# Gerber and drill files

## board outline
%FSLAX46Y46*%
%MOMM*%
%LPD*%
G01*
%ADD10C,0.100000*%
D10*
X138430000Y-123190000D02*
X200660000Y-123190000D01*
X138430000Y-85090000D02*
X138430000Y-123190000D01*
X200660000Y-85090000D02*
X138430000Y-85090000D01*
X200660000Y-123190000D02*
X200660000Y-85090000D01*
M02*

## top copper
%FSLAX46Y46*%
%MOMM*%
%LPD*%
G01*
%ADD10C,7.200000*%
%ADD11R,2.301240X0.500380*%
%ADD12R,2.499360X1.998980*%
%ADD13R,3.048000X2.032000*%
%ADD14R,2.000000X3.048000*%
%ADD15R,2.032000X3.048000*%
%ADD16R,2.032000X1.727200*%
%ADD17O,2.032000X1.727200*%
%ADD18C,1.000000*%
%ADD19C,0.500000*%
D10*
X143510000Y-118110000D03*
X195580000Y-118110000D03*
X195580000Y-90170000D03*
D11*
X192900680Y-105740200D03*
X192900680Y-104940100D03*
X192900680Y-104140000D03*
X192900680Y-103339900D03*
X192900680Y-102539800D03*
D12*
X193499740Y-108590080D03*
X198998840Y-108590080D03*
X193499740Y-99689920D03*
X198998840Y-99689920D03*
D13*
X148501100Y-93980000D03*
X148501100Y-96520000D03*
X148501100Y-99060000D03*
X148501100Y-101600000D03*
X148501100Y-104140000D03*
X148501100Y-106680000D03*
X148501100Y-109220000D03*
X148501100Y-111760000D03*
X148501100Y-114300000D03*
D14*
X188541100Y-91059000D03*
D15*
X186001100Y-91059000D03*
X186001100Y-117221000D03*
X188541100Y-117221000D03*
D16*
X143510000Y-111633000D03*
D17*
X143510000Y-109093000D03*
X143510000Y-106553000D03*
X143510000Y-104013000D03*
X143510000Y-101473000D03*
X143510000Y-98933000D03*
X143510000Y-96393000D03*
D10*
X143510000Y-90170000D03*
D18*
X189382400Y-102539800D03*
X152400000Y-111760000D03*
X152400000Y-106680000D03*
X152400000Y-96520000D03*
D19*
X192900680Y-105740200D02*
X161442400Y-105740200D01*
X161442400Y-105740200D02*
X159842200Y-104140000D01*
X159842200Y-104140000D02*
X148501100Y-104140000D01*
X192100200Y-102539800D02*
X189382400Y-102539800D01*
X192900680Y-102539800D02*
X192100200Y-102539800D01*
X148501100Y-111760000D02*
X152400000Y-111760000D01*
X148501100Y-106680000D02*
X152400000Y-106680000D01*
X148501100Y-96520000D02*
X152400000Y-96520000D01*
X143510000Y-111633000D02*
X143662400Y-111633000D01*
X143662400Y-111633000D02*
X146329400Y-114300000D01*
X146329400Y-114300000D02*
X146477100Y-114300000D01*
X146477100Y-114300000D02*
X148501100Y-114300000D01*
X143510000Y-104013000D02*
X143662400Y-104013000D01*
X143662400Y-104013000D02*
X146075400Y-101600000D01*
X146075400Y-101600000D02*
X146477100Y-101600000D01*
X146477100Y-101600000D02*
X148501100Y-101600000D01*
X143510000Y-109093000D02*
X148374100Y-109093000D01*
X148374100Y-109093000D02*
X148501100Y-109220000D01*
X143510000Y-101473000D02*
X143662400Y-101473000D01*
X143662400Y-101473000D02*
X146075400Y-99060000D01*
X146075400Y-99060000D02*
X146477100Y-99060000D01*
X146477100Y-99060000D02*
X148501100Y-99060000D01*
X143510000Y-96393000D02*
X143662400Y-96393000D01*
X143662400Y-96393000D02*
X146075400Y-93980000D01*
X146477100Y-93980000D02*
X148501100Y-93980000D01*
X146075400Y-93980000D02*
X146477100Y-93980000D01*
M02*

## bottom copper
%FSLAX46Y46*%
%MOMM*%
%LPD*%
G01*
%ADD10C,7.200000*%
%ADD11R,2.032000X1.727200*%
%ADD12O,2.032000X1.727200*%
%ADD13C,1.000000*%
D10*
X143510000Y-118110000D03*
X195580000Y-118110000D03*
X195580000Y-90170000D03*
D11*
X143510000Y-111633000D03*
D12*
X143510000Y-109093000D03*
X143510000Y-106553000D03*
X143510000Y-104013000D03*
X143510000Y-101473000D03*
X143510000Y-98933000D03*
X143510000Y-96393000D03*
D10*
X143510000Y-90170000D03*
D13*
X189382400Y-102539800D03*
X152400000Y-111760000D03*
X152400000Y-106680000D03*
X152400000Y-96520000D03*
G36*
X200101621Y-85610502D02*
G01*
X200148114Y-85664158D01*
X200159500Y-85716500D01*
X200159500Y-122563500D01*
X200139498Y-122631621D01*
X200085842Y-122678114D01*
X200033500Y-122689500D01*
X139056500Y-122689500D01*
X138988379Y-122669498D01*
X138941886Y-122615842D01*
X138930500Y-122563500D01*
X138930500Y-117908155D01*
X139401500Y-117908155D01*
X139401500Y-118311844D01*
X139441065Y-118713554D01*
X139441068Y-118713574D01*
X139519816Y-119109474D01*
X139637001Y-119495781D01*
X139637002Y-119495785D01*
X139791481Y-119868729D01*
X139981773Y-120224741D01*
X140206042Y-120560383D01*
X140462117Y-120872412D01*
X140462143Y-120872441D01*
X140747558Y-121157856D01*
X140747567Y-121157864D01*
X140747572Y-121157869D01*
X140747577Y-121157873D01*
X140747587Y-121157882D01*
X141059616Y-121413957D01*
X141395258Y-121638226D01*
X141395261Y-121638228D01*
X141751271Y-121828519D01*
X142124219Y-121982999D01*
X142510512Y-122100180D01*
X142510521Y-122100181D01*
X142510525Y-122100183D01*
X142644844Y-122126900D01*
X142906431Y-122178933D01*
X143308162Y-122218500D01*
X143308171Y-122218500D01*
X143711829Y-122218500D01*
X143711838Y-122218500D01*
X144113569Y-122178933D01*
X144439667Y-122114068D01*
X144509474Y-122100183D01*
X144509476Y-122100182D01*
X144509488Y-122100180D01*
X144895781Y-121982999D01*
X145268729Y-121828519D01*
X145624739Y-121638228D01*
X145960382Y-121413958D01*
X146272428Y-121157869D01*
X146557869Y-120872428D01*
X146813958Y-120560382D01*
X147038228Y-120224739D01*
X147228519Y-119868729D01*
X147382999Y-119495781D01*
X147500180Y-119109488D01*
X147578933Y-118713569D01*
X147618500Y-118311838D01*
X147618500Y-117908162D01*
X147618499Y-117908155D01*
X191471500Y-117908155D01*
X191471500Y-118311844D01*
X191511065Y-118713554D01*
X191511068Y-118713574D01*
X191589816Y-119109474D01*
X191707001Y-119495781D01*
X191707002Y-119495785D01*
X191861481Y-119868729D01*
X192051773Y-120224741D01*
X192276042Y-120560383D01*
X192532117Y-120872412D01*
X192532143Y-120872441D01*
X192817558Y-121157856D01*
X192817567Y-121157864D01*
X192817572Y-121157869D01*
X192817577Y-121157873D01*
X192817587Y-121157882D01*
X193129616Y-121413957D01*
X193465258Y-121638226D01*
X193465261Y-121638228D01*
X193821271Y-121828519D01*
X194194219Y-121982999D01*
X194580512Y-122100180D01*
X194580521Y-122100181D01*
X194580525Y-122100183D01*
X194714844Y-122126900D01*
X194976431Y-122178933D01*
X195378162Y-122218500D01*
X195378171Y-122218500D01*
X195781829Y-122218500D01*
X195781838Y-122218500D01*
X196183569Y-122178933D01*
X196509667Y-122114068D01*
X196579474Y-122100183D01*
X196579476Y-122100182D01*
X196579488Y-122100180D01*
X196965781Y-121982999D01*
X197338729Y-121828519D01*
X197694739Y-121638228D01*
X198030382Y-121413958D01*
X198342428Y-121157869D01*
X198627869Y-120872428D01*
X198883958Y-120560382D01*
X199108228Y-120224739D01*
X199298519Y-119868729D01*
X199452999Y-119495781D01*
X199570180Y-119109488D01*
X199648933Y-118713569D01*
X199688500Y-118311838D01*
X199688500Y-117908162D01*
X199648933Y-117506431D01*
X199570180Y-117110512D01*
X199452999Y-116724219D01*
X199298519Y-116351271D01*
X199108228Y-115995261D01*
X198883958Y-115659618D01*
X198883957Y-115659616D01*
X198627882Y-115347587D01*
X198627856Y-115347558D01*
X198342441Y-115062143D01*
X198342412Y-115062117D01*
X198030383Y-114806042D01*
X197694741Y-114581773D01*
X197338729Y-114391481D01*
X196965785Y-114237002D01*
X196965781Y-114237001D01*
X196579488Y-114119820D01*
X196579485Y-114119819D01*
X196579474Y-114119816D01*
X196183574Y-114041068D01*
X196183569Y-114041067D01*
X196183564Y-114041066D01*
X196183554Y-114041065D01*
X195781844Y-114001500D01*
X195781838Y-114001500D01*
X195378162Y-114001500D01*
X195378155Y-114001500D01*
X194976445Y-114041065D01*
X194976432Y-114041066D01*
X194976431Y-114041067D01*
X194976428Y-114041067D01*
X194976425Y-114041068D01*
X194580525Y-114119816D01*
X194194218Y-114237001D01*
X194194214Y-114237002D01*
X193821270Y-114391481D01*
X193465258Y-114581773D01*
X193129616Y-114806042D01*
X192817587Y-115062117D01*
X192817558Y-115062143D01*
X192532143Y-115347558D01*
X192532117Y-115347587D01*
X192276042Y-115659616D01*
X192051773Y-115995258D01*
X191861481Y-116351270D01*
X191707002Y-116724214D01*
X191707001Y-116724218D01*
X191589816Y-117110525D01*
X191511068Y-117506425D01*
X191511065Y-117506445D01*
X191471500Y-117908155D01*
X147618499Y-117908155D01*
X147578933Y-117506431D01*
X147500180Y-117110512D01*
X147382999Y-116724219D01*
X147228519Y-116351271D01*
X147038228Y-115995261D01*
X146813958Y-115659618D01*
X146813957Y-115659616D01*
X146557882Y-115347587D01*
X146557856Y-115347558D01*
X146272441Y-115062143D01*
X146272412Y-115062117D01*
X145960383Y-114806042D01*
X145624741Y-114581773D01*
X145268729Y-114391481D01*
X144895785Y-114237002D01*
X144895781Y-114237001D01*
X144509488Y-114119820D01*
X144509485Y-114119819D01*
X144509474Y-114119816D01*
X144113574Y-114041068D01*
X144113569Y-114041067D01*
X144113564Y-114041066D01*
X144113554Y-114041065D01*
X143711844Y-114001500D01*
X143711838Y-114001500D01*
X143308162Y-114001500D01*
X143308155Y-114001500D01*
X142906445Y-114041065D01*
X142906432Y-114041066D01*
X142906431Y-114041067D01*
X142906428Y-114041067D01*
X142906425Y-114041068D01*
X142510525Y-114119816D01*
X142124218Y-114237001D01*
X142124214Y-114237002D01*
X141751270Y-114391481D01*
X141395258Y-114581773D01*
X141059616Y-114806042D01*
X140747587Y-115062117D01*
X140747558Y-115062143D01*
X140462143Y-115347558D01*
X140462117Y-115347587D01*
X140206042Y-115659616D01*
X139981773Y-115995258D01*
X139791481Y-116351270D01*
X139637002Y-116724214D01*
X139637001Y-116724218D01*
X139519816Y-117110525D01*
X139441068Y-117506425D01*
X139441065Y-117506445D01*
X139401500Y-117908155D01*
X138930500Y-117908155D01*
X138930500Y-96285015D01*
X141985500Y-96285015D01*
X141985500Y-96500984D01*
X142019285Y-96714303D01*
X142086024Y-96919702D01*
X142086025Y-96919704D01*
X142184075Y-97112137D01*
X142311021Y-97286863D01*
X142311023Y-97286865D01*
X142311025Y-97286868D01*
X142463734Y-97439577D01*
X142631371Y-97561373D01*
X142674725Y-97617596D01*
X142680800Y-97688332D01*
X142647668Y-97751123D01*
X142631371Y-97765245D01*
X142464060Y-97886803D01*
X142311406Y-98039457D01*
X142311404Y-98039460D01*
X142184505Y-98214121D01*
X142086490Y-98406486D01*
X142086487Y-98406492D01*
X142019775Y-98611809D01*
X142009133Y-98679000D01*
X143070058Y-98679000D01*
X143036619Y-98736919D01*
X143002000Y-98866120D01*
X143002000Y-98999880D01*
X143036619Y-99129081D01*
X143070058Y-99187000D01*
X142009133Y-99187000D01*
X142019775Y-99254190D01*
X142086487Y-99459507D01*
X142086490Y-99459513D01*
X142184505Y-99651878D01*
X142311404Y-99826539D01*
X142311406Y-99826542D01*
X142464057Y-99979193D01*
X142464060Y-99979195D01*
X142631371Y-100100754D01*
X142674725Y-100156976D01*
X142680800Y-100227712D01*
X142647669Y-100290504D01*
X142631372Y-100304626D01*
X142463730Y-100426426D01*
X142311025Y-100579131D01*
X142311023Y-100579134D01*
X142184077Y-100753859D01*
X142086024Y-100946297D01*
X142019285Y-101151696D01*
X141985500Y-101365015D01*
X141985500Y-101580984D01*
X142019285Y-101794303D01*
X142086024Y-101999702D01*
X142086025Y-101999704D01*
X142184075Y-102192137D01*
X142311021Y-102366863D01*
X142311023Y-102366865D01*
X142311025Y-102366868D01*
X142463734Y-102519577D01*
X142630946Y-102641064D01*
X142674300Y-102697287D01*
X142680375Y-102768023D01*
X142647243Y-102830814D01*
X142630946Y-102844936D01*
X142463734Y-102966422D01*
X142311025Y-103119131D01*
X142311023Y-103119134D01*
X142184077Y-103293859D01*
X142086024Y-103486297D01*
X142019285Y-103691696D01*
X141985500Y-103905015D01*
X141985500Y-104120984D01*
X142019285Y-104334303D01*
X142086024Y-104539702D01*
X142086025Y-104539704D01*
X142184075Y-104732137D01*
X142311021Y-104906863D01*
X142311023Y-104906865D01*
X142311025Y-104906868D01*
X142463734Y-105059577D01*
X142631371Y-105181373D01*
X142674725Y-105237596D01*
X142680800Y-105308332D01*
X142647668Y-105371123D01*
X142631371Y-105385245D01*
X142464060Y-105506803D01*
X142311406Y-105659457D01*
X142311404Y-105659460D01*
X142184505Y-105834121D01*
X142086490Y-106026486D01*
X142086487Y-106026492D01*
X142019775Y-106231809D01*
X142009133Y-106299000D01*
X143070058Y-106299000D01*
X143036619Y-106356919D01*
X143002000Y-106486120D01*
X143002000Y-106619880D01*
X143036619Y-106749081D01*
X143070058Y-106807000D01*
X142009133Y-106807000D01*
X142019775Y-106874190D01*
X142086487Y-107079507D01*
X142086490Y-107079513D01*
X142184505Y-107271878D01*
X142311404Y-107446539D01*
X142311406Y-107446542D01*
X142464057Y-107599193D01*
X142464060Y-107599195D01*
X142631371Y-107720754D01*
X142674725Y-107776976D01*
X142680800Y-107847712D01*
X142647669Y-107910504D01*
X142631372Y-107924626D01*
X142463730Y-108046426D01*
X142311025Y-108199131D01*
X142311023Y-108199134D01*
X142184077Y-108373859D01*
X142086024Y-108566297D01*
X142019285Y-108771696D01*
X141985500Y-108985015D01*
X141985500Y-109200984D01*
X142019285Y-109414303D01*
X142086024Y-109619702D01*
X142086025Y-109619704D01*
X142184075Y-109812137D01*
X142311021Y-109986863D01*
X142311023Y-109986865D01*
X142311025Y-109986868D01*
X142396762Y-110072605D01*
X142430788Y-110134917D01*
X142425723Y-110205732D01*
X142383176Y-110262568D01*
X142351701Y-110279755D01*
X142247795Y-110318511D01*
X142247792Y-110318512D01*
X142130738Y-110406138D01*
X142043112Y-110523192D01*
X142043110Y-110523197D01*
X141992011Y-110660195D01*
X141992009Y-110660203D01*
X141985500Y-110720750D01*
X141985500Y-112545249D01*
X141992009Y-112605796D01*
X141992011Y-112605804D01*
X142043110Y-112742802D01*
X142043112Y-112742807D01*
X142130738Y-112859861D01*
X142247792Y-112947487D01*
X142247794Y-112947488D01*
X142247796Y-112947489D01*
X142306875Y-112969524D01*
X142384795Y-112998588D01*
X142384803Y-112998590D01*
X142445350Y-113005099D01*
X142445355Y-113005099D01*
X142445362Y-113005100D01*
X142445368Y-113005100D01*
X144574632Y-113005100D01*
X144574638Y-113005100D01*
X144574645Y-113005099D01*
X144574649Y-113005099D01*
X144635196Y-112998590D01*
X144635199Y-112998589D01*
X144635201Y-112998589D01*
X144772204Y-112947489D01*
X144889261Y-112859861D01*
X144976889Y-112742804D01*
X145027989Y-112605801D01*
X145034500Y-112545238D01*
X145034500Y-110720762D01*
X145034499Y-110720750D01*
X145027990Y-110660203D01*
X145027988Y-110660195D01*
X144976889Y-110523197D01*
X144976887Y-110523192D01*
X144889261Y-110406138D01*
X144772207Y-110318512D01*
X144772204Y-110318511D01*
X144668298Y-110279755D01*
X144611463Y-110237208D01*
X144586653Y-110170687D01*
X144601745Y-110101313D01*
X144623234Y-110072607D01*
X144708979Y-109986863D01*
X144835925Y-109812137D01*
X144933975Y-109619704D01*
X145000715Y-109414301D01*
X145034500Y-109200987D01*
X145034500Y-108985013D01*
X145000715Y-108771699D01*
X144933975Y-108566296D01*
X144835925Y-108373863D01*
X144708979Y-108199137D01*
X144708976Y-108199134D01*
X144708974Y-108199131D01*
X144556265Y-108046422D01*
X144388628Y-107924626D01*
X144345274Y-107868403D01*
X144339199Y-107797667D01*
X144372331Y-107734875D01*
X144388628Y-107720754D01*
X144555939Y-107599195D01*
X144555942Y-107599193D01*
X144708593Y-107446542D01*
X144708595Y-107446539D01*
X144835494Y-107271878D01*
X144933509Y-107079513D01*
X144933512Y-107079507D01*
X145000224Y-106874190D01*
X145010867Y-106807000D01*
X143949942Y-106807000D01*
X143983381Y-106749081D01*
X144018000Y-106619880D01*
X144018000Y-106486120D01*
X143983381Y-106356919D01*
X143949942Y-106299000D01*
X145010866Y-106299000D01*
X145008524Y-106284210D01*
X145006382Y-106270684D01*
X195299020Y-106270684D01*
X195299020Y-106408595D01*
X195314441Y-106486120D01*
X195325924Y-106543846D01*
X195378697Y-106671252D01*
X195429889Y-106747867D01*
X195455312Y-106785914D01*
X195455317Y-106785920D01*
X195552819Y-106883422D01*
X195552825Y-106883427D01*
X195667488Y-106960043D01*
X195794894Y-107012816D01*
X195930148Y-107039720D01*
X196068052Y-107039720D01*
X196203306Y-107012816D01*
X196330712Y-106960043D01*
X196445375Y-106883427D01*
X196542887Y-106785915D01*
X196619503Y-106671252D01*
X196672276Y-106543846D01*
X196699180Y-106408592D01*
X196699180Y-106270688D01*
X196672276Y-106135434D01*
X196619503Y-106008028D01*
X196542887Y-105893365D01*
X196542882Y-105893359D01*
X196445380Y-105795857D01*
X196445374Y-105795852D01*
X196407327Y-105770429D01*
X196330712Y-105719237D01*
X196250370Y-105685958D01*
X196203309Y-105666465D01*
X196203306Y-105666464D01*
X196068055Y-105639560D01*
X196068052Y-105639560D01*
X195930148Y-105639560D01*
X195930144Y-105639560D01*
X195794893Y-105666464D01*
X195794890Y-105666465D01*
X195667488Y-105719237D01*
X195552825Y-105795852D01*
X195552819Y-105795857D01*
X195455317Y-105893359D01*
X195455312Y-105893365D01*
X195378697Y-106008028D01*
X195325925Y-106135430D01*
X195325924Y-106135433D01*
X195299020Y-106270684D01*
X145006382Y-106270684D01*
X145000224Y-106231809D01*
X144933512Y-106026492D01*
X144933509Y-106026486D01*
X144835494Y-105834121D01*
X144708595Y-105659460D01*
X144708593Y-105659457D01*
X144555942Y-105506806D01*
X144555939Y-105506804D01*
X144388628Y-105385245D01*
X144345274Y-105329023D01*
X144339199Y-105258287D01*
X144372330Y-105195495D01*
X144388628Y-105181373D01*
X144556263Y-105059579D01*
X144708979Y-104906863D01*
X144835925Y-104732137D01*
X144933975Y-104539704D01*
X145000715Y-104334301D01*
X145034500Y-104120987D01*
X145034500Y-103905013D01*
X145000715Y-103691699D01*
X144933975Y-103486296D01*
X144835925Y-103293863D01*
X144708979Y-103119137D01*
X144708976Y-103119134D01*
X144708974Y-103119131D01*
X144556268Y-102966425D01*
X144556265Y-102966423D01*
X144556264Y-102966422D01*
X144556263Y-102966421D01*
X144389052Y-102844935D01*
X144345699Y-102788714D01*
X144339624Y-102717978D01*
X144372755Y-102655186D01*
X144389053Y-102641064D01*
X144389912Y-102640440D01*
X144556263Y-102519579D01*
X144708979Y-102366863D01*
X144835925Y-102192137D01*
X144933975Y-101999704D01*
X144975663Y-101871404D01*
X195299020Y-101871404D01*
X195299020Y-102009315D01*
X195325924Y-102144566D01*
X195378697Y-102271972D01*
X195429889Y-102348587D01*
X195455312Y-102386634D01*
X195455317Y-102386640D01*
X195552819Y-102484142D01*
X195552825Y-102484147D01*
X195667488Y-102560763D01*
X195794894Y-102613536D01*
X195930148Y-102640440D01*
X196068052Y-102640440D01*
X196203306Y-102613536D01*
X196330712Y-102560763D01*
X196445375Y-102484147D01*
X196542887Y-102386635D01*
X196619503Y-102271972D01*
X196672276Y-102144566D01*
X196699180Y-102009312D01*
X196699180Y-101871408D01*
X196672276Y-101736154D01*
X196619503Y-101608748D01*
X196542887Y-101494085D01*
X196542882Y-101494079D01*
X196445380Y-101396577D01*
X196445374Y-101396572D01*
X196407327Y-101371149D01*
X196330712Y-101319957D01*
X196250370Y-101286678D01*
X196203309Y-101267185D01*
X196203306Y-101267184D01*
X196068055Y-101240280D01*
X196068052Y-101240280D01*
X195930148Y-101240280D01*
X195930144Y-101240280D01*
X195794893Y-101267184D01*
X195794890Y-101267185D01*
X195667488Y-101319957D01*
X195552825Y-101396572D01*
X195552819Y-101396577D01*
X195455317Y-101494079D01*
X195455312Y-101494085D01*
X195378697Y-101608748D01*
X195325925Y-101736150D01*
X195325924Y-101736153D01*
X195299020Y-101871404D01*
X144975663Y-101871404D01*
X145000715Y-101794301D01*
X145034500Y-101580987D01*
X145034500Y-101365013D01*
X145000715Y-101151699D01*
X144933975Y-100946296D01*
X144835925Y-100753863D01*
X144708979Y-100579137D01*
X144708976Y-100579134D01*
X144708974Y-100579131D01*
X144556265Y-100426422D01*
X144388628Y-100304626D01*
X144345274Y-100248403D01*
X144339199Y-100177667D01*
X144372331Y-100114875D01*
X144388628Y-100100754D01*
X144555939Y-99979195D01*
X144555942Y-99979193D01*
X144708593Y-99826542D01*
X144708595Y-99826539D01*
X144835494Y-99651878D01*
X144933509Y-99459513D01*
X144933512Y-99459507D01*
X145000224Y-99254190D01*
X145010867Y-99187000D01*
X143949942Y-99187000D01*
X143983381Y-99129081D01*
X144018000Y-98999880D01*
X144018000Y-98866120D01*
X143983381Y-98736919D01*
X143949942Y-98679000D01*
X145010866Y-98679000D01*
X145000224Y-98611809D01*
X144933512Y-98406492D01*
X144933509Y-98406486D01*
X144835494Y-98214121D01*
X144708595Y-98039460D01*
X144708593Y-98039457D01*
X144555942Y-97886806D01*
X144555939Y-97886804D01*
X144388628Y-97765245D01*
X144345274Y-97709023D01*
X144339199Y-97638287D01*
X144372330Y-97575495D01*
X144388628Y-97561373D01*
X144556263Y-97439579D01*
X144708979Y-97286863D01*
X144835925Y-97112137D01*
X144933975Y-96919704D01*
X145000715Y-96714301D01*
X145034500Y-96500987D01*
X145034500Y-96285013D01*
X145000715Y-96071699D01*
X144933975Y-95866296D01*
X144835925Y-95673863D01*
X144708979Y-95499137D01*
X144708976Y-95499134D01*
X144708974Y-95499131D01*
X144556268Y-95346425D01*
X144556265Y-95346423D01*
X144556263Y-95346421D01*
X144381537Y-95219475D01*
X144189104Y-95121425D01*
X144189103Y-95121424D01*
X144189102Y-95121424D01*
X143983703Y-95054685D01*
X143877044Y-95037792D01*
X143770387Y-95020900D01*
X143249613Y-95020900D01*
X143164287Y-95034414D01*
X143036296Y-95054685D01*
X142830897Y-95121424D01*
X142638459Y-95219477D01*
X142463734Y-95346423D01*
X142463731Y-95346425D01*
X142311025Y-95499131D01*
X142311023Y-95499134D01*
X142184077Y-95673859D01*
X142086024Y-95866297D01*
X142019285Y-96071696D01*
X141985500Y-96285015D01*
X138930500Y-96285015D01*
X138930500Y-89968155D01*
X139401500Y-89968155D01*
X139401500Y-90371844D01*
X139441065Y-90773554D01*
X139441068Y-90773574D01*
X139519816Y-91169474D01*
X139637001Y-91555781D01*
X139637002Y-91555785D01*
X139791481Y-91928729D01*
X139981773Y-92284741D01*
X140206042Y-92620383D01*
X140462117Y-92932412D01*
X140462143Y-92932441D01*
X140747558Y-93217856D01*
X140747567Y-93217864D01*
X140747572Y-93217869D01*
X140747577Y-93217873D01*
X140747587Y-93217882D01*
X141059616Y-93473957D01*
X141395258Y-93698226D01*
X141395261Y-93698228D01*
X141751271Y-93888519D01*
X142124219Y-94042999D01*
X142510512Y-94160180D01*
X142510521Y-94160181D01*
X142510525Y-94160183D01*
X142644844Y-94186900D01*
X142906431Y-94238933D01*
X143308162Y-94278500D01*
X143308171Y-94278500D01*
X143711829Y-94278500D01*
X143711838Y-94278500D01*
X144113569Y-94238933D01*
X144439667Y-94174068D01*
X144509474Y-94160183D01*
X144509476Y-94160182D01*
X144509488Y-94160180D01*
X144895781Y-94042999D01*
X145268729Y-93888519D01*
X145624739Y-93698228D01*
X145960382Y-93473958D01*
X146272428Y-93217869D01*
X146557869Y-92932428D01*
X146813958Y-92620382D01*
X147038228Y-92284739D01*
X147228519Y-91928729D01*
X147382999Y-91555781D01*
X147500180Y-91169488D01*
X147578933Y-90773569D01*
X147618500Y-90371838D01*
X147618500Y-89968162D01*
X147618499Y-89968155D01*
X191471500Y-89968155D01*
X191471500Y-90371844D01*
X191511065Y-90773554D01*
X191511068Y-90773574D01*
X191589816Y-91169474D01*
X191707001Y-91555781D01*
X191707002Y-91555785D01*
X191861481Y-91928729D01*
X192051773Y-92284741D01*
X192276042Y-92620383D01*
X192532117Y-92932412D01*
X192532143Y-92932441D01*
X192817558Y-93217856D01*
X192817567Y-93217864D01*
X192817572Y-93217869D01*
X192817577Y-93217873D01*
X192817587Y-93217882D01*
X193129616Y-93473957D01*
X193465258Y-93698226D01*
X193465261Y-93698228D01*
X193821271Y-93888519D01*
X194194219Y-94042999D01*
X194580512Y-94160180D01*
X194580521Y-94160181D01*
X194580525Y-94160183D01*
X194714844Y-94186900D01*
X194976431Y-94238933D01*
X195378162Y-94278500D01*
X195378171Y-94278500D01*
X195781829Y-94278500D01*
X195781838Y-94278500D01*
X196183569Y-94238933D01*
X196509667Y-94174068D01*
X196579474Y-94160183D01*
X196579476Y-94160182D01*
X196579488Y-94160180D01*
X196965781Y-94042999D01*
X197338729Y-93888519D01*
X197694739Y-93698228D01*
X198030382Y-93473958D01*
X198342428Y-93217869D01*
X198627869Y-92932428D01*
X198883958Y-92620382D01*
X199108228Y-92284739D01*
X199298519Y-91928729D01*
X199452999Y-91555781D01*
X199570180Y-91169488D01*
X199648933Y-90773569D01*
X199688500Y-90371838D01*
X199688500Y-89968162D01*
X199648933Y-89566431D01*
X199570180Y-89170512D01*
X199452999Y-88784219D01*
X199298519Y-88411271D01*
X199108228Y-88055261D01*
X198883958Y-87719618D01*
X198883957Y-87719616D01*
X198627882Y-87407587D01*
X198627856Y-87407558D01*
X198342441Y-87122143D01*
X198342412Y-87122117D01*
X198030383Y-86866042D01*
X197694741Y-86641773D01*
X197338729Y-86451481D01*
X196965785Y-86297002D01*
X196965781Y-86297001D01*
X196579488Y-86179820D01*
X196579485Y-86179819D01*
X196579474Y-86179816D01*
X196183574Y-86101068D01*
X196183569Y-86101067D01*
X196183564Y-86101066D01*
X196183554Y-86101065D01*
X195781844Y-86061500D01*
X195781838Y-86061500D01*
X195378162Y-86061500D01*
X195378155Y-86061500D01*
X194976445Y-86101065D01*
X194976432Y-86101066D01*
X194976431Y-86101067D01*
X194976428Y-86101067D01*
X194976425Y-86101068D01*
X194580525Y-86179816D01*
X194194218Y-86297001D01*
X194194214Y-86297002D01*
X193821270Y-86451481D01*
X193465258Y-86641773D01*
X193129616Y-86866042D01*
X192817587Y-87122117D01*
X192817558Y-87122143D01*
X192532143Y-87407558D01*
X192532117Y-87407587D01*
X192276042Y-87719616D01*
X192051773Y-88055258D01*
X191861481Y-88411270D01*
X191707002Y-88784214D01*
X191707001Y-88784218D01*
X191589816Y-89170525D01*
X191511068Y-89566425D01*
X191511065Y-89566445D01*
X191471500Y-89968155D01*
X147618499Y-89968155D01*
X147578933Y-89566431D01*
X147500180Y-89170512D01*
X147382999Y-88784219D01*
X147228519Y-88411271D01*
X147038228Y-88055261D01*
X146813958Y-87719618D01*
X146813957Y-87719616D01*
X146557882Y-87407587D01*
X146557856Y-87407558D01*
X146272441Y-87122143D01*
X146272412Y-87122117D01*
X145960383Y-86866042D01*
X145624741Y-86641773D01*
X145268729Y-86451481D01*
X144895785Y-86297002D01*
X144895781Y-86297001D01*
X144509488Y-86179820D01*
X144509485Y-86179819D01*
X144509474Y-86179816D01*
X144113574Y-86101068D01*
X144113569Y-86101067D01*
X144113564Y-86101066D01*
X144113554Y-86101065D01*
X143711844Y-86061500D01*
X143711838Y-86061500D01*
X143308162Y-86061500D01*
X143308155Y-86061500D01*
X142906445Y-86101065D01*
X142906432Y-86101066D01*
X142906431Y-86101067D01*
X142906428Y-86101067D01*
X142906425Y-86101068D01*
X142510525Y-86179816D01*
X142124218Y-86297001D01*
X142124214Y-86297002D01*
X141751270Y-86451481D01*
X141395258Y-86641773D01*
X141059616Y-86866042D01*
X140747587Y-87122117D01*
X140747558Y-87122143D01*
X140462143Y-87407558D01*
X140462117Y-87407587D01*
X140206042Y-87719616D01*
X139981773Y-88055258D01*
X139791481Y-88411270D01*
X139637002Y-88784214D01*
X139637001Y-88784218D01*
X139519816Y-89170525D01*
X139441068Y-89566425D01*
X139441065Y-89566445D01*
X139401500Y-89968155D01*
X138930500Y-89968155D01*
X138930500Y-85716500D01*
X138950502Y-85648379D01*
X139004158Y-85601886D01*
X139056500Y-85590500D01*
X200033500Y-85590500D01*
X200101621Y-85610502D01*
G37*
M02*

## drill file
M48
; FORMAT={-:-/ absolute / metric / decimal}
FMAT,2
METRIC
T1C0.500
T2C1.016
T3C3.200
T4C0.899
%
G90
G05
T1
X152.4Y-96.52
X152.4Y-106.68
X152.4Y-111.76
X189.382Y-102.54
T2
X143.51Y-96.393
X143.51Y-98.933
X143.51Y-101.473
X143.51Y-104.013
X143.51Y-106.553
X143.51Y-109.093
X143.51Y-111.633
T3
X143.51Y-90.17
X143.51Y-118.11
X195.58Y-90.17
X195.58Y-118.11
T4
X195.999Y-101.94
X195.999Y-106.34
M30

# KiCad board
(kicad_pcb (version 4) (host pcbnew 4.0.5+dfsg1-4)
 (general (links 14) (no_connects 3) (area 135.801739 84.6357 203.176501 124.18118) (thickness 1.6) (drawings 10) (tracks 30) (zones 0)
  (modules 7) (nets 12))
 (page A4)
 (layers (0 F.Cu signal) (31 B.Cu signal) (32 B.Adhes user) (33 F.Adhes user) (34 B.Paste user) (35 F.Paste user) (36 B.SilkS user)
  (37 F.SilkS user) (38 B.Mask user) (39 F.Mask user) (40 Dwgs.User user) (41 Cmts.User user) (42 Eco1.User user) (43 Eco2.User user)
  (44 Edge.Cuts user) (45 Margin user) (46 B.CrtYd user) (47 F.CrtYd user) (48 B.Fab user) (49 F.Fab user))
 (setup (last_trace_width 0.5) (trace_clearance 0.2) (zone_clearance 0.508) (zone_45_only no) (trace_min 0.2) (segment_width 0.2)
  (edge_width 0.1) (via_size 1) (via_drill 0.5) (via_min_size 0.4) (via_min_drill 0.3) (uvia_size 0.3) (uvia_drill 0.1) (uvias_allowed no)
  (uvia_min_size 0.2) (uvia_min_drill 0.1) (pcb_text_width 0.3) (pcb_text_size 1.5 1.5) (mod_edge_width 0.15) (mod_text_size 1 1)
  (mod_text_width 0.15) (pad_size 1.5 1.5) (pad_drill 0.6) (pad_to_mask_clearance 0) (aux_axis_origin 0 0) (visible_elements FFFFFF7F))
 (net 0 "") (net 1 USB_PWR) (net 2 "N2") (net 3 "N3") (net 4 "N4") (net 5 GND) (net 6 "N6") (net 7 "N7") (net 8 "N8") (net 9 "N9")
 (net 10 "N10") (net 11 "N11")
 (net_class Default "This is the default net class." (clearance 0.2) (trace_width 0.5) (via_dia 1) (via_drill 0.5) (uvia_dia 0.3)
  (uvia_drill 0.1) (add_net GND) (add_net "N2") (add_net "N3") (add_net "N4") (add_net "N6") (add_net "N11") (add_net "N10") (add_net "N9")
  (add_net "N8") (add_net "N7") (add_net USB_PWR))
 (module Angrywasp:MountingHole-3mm (layer F.Cu) (at 143.51 118.11)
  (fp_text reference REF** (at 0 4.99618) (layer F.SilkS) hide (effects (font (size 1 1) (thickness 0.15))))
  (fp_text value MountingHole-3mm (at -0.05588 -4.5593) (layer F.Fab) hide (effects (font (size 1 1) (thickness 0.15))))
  (pad 1 thru_hole circle (at 0 0) (size 7.2 7.2) (drill 3.2) (layers *.Cu *.Mask)))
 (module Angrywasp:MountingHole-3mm (layer F.Cu) (at 195.58 118.11)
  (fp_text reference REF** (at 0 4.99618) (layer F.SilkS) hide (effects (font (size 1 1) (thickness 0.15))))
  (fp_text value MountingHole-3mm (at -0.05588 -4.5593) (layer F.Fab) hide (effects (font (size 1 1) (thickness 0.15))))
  (pad 1 thru_hole circle (at 0 0) (size 7.2 7.2) (drill 3.2) (layers *.Cu *.Mask)))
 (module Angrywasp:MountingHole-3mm (layer F.Cu) (at 195.58 90.17)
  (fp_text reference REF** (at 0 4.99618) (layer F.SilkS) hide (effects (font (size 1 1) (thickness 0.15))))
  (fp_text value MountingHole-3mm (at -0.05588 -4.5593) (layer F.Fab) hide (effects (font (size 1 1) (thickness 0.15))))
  (pad 1 thru_hole circle (at 0 0) (size 7.2 7.2) (drill 3.2) (layers *.Cu *.Mask)))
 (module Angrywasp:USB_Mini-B (layer F.Cu) (at 196.85 104.14 180)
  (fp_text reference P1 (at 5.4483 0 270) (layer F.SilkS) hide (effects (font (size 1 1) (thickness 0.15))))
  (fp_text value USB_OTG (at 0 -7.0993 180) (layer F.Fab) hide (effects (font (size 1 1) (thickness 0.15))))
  (pad 1 smd rect (at 3.94932 -1.6002 180) (size 2.30124 0.50038) (layers F.Cu F.Paste F.Mask) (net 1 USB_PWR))
  (pad 2 smd rect (at 3.94932 -0.8001 180) (size 2.30124 0.50038) (layers F.Cu F.Paste F.Mask) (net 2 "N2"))
  (pad 3 smd rect (at 3.94932 0 180) (size 2.30124 0.50038) (layers F.Cu F.Paste F.Mask) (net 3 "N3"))
  (pad 4 smd rect (at 3.94932 0.8001 180) (size 2.30124 0.50038) (layers F.Cu F.Paste F.Mask) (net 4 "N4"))
  (pad 5 smd rect (at 3.94932 1.6002 180) (size 2.30124 0.50038) (layers F.Cu F.Paste F.Mask) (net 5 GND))
  (pad 6 smd rect (at 3.35026 -4.45008 180) (size 2.49936 1.99898) (layers F.Cu F.Paste F.Mask) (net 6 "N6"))
  (pad 6 smd rect (at -2.14884 -4.45008 180) (size 2.49936 1.99898) (layers F.Cu F.Paste F.Mask) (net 6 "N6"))
  (pad 6 smd rect (at 3.35026 4.45008 180) (size 2.49936 1.99898) (layers F.Cu F.Paste F.Mask) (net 6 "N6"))
  (pad 6 smd rect (at -2.14884 4.45008 180) (size 2.49936 1.99898) (layers F.Cu F.Paste F.Mask) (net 6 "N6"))
  (pad "" np_thru_hole circle (at 0.8509 -2.19964 180) (size 0.89916 0.89916) (drill 0.89916) (layers *.Cu *.Mask F.SilkS))
  (pad "" np_thru_hole circle (at 0.8509 2.19964 180) (size 0.89916 0.89916) (drill 0.89916) (layers *.Cu *.Mask F.SilkS)))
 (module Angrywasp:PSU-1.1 (layer F.Cu) (at 148.5011 104.14)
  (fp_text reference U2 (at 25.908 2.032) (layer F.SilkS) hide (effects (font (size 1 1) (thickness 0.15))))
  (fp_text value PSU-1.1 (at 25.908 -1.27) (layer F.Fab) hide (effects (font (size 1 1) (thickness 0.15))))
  (pad 1 smd rect (at 0 -10.16) (size 3.048 2.032) (layers F.Cu F.Paste F.Mask) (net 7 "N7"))
  (pad 2 smd rect (at 0 -7.62) (size 3.048 2.032) (layers F.Cu F.Paste F.Mask) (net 5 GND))
  (pad 3 smd rect (at 0 -5.08) (size 3.048 2.032) (layers F.Cu F.Paste F.Mask) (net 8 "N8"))
  (pad 4 smd rect (at 0 -2.54) (size 3.048 2.032) (layers F.Cu F.Paste F.Mask) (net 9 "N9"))
  (pad 5 smd rect (at 0 0) (size 3.048 2.032) (layers F.Cu F.Paste F.Mask) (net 1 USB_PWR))
  (pad 6 smd rect (at 0 2.54) (size 3.048 2.032) (layers F.Cu F.Paste F.Mask) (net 5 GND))
  (pad 7 smd rect (at 0 5.08) (size 3.048 2.032) (layers F.Cu F.Paste F.Mask) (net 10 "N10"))
  (pad 8 smd rect (at 0 7.62) (size 3.048 2.032) (layers F.Cu F.Paste F.Mask) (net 5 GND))
  (pad 9 smd rect (at 0 10.16) (size 3.048 2.032) (layers F.Cu F.Paste F.Mask) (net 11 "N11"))
  (pad "" smd rect (at 40.04 -13.081 90) (size 3.048 2) (layers F.Cu F.Paste F.Mask))
  (pad "" smd rect (at 37.5 -13.081 90) (size 3.048 2.032) (layers F.Cu F.Paste F.Mask))
  (pad "" smd rect (at 37.5 13.081 90) (size 3.048 2.032) (layers F.Cu F.Paste F.Mask))
  (pad "" smd rect (at 40.04 13.081 90) (size 3.048 2.032) (layers F.Cu F.Paste F.Mask)))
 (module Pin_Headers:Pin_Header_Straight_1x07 (layer F.Cu) (at 143.51 111.633 180)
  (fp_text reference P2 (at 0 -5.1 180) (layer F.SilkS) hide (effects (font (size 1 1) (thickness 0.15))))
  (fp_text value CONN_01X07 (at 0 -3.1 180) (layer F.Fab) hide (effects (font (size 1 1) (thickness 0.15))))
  (pad 1 thru_hole rect (at 0 0 180) (size 2.032 1.7272) (drill 1.016) (layers *.Cu *.Mask) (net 11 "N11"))
  (pad 2 thru_hole oval (at 0 2.54 180) (size 2.032 1.7272) (drill 1.016) (layers *.Cu *.Mask) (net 10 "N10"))
  (pad 3 thru_hole oval (at 0 5.08 180) (size 2.032 1.7272) (drill 1.016) (layers *.Cu *.Mask) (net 5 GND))
  (pad 4 thru_hole oval (at 0 7.62 180) (size 2.032 1.7272) (drill 1.016) (layers *.Cu *.Mask) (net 9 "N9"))
  (pad 5 thru_hole oval (at 0 10.16 180) (size 2.032 1.7272) (drill 1.016) (layers *.Cu *.Mask) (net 8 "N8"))
  (pad 6 thru_hole oval (at 0 12.7 180) (size 2.032 1.7272) (drill 1.016) (layers *.Cu *.Mask) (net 5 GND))
  (pad 7 thru_hole oval (at 0 15.24 180) (size 2.032 1.7272) (drill 1.016) (layers *.Cu *.Mask) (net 7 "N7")))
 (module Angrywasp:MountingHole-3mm (layer F.Cu) (at 143.51 90.17)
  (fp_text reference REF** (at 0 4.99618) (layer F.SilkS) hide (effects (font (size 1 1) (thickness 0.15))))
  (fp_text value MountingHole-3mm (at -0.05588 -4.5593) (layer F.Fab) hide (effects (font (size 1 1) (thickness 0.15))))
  (pad 1 thru_hole circle (at 0 0) (size 7.2 7.2) (drill 3.2) (layers *.Cu *.Mask)))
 (gr_line (start 138.43 123.19) (end 200.66 123.19) (layer Edge.Cuts) (width 0.1))
 (gr_line (start 138.43 85.09) (end 138.43 123.19) (layer Edge.Cuts) (width 0.1))
 (gr_line (start 200.66 85.09) (end 138.43 85.09) (layer Edge.Cuts) (width 0.1))
 (gr_line (start 200.66 123.19) (end 200.66 85.09) (layer Edge.Cuts) (width 0.1))
 (segment (start 192.90068 105.7402) (end 161.4424 105.7402) (width 0.5) (layer F.Cu) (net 1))
 (segment (start 161.4424 105.7402) (end 159.8422 104.14) (width 0.5) (layer F.Cu) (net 1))
 (segment (start 159.8422 104.14) (end 148.5011 104.14) (width 0.5) (layer F.Cu) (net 1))
 (segment (start 192.1002 102.5398) (end 189.3824 102.5398) (width 0.5) (layer F.Cu) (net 5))
 (via (at 189.3824 102.5398) (size 1) (drill 0.5) (layers F.Cu B.Cu) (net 5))
 (segment (start 192.90068 102.5398) (end 192.1002 102.5398) (width 0.5) (layer F.Cu) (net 5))
 (via (at 152.4 111.76) (size 1) (drill 0.5) (layers F.Cu B.Cu) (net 5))
 (segment (start 148.5011 111.76) (end 152.4 111.76) (width 0.5) (layer F.Cu) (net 5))
 (via (at 152.4 106.68) (size 1) (drill 0.5) (layers F.Cu B.Cu) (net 5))
 (segment (start 148.5011 106.68) (end 152.4 106.68) (width 0.5) (layer F.Cu) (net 5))
 (via (at 152.4 96.52) (size 1) (drill 0.5) (layers F.Cu B.Cu) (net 5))
 (segment (start 148.5011 96.52) (end 152.4 96.52) (width 0.5) (layer F.Cu) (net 5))
 (segment (start 143.51 111.633) (end 143.6624 111.633) (width 0.5) (layer F.Cu) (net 11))
 (segment (start 143.6624 111.633) (end 146.3294 114.3) (width 0.5) (layer F.Cu) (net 11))
 (segment (start 146.3294 114.3) (end 146.4771 114.3) (width 0.5) (layer F.Cu) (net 11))
 (segment (start 146.4771 114.3) (end 148.5011 114.3) (width 0.5) (layer F.Cu) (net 11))
 (segment (start 143.51 104.013) (end 143.6624 104.013) (width 0.5) (layer F.Cu) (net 9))
 (segment (start 143.6624 104.013) (end 146.0754 101.6) (width 0.5) (layer F.Cu) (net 9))
 (segment (start 146.0754 101.6) (end 146.4771 101.6) (width 0.5) (layer F.Cu) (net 9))
 (segment (start 146.4771 101.6) (end 148.5011 101.6) (width 0.5) (layer F.Cu) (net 9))
 (segment (start 143.51 109.093) (end 148.3741 109.093) (width 0.5) (layer F.Cu) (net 10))
 (segment (start 148.3741 109.093) (end 148.5011 109.22) (width 0.5) (layer F.Cu) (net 10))
 (segment (start 143.51 101.473) (end 143.6624 101.473) (width 0.5) (layer F.Cu) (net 8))
 (segment (start 143.6624 101.473) (end 146.0754 99.06) (width 0.5) (layer F.Cu) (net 8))
 (segment (start 146.0754 99.06) (end 146.4771 99.06) (width 0.5) (layer F.Cu) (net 8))
 (segment (start 146.4771 99.06) (end 148.5011 99.06) (width 0.5) (layer F.Cu) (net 8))
 (segment (start 143.51 96.393) (end 143.6624 96.393) (width 0.5) (layer F.Cu) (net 7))
 (segment (start 143.6624 96.393) (end 146.0754 93.98) (width 0.5) (layer F.Cu) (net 7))
 (segment (start 146.4771 93.98) (end 148.5011 93.98) (width 0.5) (layer F.Cu) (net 7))
 (segment (start 146.0754 93.98) (end 146.4771 93.98) (width 0.5) (layer F.Cu) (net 7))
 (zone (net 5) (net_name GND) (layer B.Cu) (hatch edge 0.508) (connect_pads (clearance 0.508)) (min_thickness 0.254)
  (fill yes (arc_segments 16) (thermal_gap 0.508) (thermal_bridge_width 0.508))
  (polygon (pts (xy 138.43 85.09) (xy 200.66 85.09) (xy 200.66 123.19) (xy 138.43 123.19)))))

